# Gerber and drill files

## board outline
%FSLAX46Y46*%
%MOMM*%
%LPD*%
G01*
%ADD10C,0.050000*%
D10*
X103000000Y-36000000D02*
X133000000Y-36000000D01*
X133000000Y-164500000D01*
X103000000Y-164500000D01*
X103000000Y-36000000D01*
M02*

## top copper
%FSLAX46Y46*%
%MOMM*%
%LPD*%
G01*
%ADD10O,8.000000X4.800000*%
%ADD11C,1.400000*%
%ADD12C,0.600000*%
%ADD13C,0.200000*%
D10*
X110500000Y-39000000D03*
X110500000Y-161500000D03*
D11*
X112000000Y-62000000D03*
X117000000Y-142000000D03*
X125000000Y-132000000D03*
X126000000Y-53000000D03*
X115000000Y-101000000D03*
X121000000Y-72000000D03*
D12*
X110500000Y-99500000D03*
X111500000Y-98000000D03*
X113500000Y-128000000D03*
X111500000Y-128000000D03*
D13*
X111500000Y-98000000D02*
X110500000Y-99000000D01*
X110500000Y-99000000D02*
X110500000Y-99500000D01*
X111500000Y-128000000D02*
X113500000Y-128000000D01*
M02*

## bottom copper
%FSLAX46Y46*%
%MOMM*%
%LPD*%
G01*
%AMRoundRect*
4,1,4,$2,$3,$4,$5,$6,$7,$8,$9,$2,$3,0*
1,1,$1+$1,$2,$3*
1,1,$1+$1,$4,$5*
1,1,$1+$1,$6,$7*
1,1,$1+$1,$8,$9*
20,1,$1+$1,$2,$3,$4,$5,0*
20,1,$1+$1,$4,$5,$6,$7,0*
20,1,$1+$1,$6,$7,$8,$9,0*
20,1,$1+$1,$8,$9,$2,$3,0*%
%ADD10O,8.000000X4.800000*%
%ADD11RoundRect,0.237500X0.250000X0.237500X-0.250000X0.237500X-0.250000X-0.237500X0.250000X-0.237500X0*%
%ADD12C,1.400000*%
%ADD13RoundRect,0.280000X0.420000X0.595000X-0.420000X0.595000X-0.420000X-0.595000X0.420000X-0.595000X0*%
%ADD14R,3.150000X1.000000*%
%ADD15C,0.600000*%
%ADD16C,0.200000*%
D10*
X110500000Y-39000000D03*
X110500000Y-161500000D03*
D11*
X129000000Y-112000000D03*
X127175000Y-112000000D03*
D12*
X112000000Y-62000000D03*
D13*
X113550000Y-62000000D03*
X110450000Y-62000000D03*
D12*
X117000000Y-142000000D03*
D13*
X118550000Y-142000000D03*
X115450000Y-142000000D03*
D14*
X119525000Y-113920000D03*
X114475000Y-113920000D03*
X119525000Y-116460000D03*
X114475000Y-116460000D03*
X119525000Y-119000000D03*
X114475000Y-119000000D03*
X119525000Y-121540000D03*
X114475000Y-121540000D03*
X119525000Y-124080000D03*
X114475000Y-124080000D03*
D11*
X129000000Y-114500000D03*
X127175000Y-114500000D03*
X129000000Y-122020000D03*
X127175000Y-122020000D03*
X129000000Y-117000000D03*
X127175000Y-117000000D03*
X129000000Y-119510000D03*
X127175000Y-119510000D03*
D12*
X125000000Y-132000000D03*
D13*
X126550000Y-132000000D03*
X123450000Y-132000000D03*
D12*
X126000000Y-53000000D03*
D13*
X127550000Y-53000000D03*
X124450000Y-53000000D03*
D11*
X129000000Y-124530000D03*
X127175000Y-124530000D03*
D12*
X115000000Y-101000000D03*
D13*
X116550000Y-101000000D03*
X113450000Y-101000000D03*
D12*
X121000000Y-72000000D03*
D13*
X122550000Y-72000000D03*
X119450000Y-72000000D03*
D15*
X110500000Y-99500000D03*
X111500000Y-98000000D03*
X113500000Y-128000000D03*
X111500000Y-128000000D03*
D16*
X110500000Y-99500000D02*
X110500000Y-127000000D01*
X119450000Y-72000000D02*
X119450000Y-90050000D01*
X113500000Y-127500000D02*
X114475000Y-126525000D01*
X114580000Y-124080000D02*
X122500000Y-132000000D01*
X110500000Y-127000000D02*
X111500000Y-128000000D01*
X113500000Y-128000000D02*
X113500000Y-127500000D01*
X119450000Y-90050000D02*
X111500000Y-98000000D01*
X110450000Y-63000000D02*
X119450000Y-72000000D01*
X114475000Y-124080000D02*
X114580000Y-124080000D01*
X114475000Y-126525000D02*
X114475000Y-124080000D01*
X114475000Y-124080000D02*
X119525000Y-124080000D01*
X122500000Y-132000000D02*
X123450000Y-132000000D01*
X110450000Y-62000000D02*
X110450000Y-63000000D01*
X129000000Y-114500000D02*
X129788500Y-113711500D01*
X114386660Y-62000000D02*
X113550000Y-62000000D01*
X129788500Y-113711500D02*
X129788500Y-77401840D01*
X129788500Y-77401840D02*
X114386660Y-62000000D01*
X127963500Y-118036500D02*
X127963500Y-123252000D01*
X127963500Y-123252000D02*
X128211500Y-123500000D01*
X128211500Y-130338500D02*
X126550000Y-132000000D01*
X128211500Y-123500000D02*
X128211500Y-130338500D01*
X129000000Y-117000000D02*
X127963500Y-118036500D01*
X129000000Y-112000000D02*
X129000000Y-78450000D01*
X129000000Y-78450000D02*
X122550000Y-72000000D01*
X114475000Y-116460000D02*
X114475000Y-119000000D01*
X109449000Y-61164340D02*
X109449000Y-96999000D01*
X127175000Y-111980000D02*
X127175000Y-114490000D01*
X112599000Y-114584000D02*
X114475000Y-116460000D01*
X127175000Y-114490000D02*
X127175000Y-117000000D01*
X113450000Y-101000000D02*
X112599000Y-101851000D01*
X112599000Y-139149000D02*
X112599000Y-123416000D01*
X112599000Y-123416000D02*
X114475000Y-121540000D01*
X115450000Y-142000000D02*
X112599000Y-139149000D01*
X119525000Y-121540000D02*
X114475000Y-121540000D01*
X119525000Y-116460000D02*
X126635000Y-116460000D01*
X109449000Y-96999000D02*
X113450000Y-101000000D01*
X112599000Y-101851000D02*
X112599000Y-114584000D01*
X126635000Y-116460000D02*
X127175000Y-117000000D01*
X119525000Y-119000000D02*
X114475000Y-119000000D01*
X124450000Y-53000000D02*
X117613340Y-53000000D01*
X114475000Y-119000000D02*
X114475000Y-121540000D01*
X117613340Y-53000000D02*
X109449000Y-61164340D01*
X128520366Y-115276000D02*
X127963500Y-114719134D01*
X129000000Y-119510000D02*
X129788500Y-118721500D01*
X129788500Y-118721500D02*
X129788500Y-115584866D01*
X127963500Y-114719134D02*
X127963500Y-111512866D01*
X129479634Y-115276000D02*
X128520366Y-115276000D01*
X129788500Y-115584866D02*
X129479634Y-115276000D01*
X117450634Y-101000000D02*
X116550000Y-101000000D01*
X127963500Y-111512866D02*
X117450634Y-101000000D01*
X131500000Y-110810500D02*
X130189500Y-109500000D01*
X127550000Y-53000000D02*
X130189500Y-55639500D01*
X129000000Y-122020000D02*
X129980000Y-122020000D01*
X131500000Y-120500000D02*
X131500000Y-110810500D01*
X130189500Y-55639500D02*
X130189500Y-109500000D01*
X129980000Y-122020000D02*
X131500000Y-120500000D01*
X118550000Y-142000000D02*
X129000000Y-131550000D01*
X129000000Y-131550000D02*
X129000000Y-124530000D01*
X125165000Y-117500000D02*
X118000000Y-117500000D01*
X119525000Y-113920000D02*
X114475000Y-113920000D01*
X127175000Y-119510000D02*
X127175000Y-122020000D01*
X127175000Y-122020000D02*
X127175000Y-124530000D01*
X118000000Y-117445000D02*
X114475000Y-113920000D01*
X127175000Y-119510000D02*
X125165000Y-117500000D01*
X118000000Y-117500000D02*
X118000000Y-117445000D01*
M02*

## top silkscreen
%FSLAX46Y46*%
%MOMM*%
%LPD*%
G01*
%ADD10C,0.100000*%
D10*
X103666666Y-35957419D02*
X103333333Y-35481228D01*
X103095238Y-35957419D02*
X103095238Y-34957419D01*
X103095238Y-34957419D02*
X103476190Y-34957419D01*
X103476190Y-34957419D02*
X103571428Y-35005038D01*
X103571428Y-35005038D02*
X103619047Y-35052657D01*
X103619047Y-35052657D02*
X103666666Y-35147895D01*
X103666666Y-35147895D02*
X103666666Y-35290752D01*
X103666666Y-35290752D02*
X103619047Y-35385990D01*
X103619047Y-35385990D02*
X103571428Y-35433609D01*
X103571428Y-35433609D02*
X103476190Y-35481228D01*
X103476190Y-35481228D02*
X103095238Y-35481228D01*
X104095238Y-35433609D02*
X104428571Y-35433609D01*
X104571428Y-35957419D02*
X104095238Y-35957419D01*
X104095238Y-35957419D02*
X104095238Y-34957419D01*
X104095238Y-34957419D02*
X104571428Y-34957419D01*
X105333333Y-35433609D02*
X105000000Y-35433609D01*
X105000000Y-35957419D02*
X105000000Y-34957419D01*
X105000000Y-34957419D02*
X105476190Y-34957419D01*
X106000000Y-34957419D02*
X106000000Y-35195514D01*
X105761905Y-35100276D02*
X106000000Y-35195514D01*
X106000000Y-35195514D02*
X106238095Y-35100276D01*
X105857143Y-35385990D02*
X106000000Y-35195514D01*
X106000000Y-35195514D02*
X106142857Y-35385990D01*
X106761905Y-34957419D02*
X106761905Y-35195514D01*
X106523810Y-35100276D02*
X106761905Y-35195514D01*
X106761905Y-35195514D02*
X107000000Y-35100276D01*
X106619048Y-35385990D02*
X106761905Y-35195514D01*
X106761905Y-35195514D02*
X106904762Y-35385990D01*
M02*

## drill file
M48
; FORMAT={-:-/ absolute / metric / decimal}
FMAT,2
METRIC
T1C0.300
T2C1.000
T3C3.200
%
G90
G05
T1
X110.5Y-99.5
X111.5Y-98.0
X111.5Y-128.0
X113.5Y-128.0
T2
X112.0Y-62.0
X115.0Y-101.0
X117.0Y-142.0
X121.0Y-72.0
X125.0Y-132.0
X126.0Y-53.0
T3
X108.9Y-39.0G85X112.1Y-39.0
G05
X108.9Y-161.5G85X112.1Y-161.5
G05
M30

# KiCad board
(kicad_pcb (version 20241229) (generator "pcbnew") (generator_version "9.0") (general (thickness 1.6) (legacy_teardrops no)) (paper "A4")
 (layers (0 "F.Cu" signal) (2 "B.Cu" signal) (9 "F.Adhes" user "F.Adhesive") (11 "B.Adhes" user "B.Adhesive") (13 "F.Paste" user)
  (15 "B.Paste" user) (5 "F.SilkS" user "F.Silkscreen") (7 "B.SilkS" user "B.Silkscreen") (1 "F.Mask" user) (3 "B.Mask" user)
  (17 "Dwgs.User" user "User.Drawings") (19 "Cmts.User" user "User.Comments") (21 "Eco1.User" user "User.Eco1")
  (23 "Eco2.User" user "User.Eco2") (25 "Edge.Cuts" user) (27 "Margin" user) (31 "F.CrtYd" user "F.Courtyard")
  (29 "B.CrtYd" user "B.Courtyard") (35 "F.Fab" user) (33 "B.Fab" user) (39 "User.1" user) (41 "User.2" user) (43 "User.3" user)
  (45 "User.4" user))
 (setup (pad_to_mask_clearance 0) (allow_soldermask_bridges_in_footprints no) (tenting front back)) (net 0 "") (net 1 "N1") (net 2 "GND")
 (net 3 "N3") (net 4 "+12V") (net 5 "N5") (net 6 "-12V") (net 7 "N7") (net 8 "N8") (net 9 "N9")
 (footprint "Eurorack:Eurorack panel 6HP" (layer "F.Cu") (at 103 36)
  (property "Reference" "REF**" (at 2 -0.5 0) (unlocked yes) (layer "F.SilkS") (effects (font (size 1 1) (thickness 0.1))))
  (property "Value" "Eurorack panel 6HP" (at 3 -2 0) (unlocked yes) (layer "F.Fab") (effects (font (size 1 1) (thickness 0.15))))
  (fp_rect (start 0 0) (end 30 128.5) (stroke (width 0.05) (type solid)) (fill no) (layer "Edge.Cuts"))
  (pad "" thru_hole oval (at 7.5 3) (size 8 4.8) (drill oval 6.4 3.2) (layers "*.Cu" "*.Mask") (remove_unused_layers no))
  (pad "" thru_hole oval (at 7.5 125.5) (size 8 4.8) (drill oval 6.4 3.2) (layers "*.Cu" "*.Mask") (remove_unused_layers no)))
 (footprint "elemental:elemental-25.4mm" (layer "B.Cu") (at 117.837802 149.513938 180)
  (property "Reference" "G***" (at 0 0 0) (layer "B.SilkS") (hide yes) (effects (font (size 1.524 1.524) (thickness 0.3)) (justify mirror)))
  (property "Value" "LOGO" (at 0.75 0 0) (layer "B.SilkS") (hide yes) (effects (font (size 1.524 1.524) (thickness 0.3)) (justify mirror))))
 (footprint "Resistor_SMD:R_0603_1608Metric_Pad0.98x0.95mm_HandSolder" (layer "B.Cu") (at 128.0875 112 180)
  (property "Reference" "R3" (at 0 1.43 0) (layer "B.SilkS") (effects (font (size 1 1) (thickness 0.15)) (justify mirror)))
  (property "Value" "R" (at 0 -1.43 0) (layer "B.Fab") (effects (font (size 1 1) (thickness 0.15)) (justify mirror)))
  (pad "1" smd roundrect (at -0.9125 0 180) (size 0.975 0.95) (layers "B.Cu" "B.Mask" "B.Paste") (roundrect_rratio 0.25) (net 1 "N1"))
  (pad "2" smd roundrect (at 0.9125 0 180) (size 0.975 0.95) (layers "B.Cu" "B.Mask" "B.Paste") (roundrect_rratio 0.25) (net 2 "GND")))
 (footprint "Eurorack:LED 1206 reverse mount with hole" (layer "B.Cu") (at 112 62 180)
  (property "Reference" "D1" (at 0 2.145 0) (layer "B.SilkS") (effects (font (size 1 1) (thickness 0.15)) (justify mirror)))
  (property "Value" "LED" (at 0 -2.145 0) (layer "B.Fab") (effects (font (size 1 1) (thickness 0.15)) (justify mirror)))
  (pad "" thru_hole circle (at 0 0 180) (size 1.4 1.4) (drill 1) (layers "*.Cu" "*.Mask") (remove_unused_layers no))
  (pad "1" smd roundrect (at -1.55 0 180) (size 1.4 1.75) (layers "B.Cu" "B.Mask" "B.Paste") (roundrect_rratio 0.2) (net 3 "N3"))
  (pad "2" smd roundrect (at 1.55 0 180) (size 1.4 1.75) (layers "B.Cu" "B.Mask" "B.Paste") (roundrect_rratio 0.2) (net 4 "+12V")))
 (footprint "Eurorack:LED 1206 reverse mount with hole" (layer "B.Cu") (at 117 142 180)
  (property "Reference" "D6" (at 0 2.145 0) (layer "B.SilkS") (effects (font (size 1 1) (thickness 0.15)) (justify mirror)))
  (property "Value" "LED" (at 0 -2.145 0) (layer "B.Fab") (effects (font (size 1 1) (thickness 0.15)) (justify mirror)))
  (pad "" thru_hole circle (at 0 0 180) (size 1.4 1.4) (drill 1) (layers "*.Cu" "*.Mask") (remove_unused_layers no))
  (pad "1" smd roundrect (at -1.55 0 180) (size 1.4 1.75) (layers "B.Cu" "B.Mask" "B.Paste") (roundrect_rratio 0.2) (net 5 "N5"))
  (pad "2" smd roundrect (at 1.55 0 180) (size 1.4 1.75) (layers "B.Cu" "B.Mask" "B.Paste") (roundrect_rratio 0.2) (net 2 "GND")))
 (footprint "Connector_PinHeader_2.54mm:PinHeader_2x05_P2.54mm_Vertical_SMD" (layer "B.Cu") (at 117 119 180)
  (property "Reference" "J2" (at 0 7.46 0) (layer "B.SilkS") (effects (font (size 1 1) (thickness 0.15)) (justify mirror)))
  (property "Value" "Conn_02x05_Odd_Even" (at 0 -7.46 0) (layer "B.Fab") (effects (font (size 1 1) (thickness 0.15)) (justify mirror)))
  (pad "1" smd rect (at -2.525 5.08 180) (size 3.15 1) (layers "B.Cu" "B.Mask" "B.Paste") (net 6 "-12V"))
  (pad "2" smd rect (at 2.525 5.08 180) (size 3.15 1) (layers "B.Cu" "B.Mask" "B.Paste") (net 6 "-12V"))
  (pad "3" smd rect (at -2.525 2.54 180) (size 3.15 1) (layers "B.Cu" "B.Mask" "B.Paste") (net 2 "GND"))
  (pad "4" smd rect (at 2.525 2.54 180) (size 3.15 1) (layers "B.Cu" "B.Mask" "B.Paste") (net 2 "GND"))
  (pad "5" smd rect (at -2.525 0 180) (size 3.15 1) (layers "B.Cu" "B.Mask" "B.Paste") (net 2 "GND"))
  (pad "6" smd rect (at 2.525 0 180) (size 3.15 1) (layers "B.Cu" "B.Mask" "B.Paste") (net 2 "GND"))
  (pad "7" smd rect (at -2.525 -2.54 180) (size 3.15 1) (layers "B.Cu" "B.Mask" "B.Paste") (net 2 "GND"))
  (pad "8" smd rect (at 2.525 -2.54 180) (size 3.15 1) (layers "B.Cu" "B.Mask" "B.Paste") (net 2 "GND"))
  (pad "9" smd rect (at -2.525 -5.08 180) (size 3.15 1) (layers "B.Cu" "B.Mask" "B.Paste") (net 4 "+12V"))
  (pad "10" smd rect (at 2.525 -5.08 180) (size 3.15 1) (layers "B.Cu" "B.Mask" "B.Paste") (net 4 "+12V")))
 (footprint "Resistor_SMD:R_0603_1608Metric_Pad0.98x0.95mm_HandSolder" (layer "B.Cu") (at 128.0875 114.5 180)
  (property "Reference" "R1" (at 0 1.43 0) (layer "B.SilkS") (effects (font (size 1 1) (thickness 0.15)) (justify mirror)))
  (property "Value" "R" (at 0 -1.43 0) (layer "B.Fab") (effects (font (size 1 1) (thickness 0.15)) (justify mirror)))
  (pad "1" smd roundrect (at -0.9125 0 180) (size 0.975 0.95) (layers "B.Cu" "B.Mask" "B.Paste") (roundrect_rratio 0.25) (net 3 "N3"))
  (pad "2" smd roundrect (at 0.9125 0 180) (size 0.975 0.95) (layers "B.Cu" "B.Mask" "B.Paste") (roundrect_rratio 0.25) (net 2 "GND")))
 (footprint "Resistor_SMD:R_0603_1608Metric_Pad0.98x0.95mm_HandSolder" (layer "B.Cu") (at 128.0875 122.02 180)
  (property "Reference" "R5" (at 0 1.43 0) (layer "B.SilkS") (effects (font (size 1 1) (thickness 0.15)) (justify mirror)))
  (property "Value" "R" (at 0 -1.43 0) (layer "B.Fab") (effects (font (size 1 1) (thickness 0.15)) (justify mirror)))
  (pad "1" smd roundrect (at -0.9125 0 180) (size 0.975 0.95) (layers "B.Cu" "B.Mask" "B.Paste") (roundrect_rratio 0.25) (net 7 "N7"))
  (pad "2" smd roundrect (at 0.9125 0 180) (size 0.975 0.95) (layers "B.Cu" "B.Mask" "B.Paste") (roundrect_rratio 0.25) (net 6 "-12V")))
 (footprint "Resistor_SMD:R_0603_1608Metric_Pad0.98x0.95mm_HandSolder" (layer "B.Cu") (at 128.0875 117 180)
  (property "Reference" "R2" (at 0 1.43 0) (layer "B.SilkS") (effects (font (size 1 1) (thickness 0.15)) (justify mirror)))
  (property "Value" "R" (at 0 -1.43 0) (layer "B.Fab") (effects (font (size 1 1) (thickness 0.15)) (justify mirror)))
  (pad "1" smd roundrect (at -0.9125 0 180) (size 0.975 0.95) (layers "B.Cu" "B.Mask" "B.Paste") (roundrect_rratio 0.25) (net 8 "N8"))
  (pad "2" smd roundrect (at 0.9125 0 180) (size 0.975 0.95) (layers "B.Cu" "B.Mask" "B.Paste") (roundrect_rratio 0.25) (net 2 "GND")))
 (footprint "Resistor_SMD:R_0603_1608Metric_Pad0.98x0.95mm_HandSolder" (layer "B.Cu") (at 128.0875 119.51 180)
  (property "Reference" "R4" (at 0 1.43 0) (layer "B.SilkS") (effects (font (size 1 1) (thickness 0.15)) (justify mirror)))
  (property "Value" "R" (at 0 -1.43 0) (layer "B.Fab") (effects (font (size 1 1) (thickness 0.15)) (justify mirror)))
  (pad "1" smd roundrect (at -0.9125 0 180) (size 0.975 0.95) (layers "B.Cu" "B.Mask" "B.Paste") (roundrect_rratio 0.25) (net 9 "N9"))
  (pad "2" smd roundrect (at 0.9125 0 180) (size 0.975 0.95) (layers "B.Cu" "B.Mask" "B.Paste") (roundrect_rratio 0.25) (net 6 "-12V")))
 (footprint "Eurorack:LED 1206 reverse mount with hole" (layer "B.Cu") (at 125 132 180)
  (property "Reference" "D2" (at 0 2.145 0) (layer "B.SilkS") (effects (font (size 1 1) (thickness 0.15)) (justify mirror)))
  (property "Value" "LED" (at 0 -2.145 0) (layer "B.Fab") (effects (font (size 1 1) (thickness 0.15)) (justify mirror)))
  (pad "" thru_hole circle (at 0 0 180) (size 1.4 1.4) (drill 1) (layers "*.Cu" "*.Mask") (remove_unused_layers no))
  (pad "1" smd roundrect (at -1.55 0 180) (size 1.4 1.75) (layers "B.Cu" "B.Mask" "B.Paste") (roundrect_rratio 0.2) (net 8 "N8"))
  (pad "2" smd roundrect (at 1.55 0 180) (size 1.4 1.75) (layers "B.Cu" "B.Mask" "B.Paste") (roundrect_rratio 0.2) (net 4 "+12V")))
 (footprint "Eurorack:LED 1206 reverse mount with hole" (layer "B.Cu") (at 126 53 180)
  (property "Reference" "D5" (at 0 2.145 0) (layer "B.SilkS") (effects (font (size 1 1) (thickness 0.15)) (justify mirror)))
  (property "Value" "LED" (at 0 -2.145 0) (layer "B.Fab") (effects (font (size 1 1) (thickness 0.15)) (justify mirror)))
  (pad "" thru_hole circle (at 0 0 180) (size 1.4 1.4) (drill 1) (layers "*.Cu" "*.Mask") (remove_unused_layers no))
  (pad "1" smd roundrect (at -1.55 0 180) (size 1.4 1.75) (layers "B.Cu" "B.Mask" "B.Paste") (roundrect_rratio 0.2) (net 7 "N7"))
  (pad "2" smd roundrect (at 1.55 0 180) (size 1.4 1.75) (layers "B.Cu" "B.Mask" "B.Paste") (roundrect_rratio 0.2) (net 2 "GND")))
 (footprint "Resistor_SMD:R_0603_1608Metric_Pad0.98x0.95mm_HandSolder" (layer "B.Cu") (at 128.0875 124.53 180)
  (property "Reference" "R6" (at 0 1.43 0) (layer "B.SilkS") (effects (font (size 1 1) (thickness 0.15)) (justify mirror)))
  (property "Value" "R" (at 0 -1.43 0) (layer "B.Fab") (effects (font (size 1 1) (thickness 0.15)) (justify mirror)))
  (pad "1" smd roundrect (at -0.9125 0 180) (size 0.975 0.95) (layers "B.Cu" "B.Mask" "B.Paste") (roundrect_rratio 0.25) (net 5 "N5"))
  (pad "2" smd roundrect (at 0.9125 0 180) (size 0.975 0.95) (layers "B.Cu" "B.Mask" "B.Paste") (roundrect_rratio 0.25) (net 6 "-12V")))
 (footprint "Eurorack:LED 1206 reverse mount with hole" (layer "B.Cu") (at 115 101 180)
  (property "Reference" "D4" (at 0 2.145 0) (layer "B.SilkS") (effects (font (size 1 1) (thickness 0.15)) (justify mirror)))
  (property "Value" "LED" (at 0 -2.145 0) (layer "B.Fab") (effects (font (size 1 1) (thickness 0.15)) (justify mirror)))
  (pad "" thru_hole circle (at 0 0 180) (size 1.4 1.4) (drill 1) (layers "*.Cu" "*.Mask") (remove_unused_layers no))
  (pad "1" smd roundrect (at -1.55 0 180) (size 1.4 1.75) (layers "B.Cu" "B.Mask" "B.Paste") (roundrect_rratio 0.2) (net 9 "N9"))
  (pad "2" smd roundrect (at 1.55 0 180) (size 1.4 1.75) (layers "B.Cu" "B.Mask" "B.Paste") (roundrect_rratio 0.2) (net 2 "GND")))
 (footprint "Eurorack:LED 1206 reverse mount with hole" (layer "B.Cu") (at 121 72 180)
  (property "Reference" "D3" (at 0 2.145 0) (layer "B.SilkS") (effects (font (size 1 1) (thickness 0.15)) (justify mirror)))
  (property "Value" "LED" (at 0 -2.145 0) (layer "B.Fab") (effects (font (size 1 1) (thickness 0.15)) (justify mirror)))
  (pad "" thru_hole circle (at 0 0 180) (size 1.4 1.4) (drill 1) (layers "*.Cu" "*.Mask") (remove_unused_layers no))
  (pad "1" smd roundrect (at -1.55 0 180) (size 1.4 1.75) (layers "B.Cu" "B.Mask" "B.Paste") (roundrect_rratio 0.2) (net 1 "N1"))
  (pad "2" smd roundrect (at 1.55 0 180) (size 1.4 1.75) (layers "B.Cu" "B.Mask" "B.Paste") (roundrect_rratio 0.2) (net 4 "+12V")))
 (segment (start 111.5 98) (end 110.5 99) (width 0.2) (layer "F.Cu") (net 4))
 (segment (start 110.5 99) (end 110.5 99.5) (width 0.2) (layer "F.Cu") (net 4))
 (segment (start 111.5 128) (end 113.5 128) (width 0.2) (layer "F.Cu") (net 4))
 (via (at 110.5 99.5) (size 0.6) (drill 0.3) (layers "F.Cu" "B.Cu") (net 4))
 (via (at 111.5 98) (size 0.6) (drill 0.3) (layers "F.Cu" "B.Cu") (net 4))
 (via (at 113.5 128) (size 0.6) (drill 0.3) (layers "F.Cu" "B.Cu") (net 4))
 (via (at 111.5 128) (size 0.6) (drill 0.3) (layers "F.Cu" "B.Cu") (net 4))
 (segment (start 110.5 99.5) (end 110.5 127) (width 0.2) (layer "B.Cu") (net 4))
 (segment (start 119.45 72) (end 119.45 90.05) (width 0.2) (layer "B.Cu") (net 4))
 (segment (start 113.5 127.5) (end 114.475 126.525) (width 0.2) (layer "B.Cu") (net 4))
 (segment (start 114.58 124.08) (end 122.5 132) (width 0.2) (layer "B.Cu") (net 4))
 (segment (start 110.5 127) (end 111.5 128) (width 0.2) (layer "B.Cu") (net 4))
 (segment (start 113.5 128) (end 113.5 127.5) (width 0.2) (layer "B.Cu") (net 4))
 (segment (start 119.45 90.05) (end 111.5 98) (width 0.2) (layer "B.Cu") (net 4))
 (segment (start 110.45 63) (end 119.45 72) (width 0.2) (layer "B.Cu") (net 4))
 (segment (start 114.475 124.08) (end 114.58 124.08) (width 0.2) (layer "B.Cu") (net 4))
 (segment (start 114.475 126.525) (end 114.475 124.08) (width 0.2) (layer "B.Cu") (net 4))
 (segment (start 114.475 124.08) (end 119.525 124.08) (width 0.2) (layer "B.Cu") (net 4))
 (segment (start 122.5 132) (end 123.45 132) (width 0.2) (layer "B.Cu") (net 4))
 (segment (start 110.45 62) (end 110.45 63) (width 0.2) (layer "B.Cu") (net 4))
 (segment (start 129 114.5) (end 129.7885 113.7115) (width 0.2) (layer "B.Cu") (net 3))
 (segment (start 114.38666 62) (end 113.55 62) (width 0.2) (layer "B.Cu") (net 3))
 (segment (start 129.7885 113.7115) (end 129.7885 77.40184) (width 0.2) (layer "B.Cu") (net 3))
 (segment (start 129.7885 77.40184) (end 114.38666 62) (width 0.2) (layer "B.Cu") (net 3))
 (segment (start 127.9635 118.0365) (end 127.9635 123.252) (width 0.2) (layer "B.Cu") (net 8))
 (segment (start 127.9635 123.252) (end 128.2115 123.5) (width 0.2) (layer "B.Cu") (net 8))
 (segment (start 128.2115 130.3385) (end 126.55 132) (width 0.2) (layer "B.Cu") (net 8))
 (segment (start 128.2115 123.5) (end 128.2115 130.3385) (width 0.2) (layer "B.Cu") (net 8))
 (segment (start 129 117) (end 127.9635 118.0365) (width 0.2) (layer "B.Cu") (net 8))
 (segment (start 129 112) (end 129 78.45) (width 0.2) (layer "B.Cu") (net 1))
 (segment (start 129 78.45) (end 122.55 72) (width 0.2) (layer "B.Cu") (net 1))
 (segment (start 114.475 116.46) (end 114.475 119) (width 0.2) (layer "B.Cu") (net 2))
 (segment (start 109.449 61.16434) (end 109.449 96.999) (width 0.2) (layer "B.Cu") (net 2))
 (segment (start 127.175 111.98) (end 127.175 114.49) (width 0.2) (layer "B.Cu") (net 2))
 (segment (start 112.599 114.584) (end 114.475 116.46) (width 0.2) (layer "B.Cu") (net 2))
 (segment (start 127.175 114.49) (end 127.175 117) (width 0.2) (layer "B.Cu") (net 2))
 (segment (start 113.45 101) (end 112.599 101.851) (width 0.2) (layer "B.Cu") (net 2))
 (segment (start 112.599 139.149) (end 112.599 123.416) (width 0.2) (layer "B.Cu") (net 2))
 (segment (start 112.599 123.416) (end 114.475 121.54) (width 0.2) (layer "B.Cu") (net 2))
 (segment (start 115.45 142) (end 112.599 139.149) (width 0.2) (layer "B.Cu") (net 2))
 (segment (start 119.525 121.54) (end 114.475 121.54) (width 0.2) (layer "B.Cu") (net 2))
 (segment (start 119.525 116.46) (end 126.635 116.46) (width 0.2) (layer "B.Cu") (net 2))
 (segment (start 109.449 96.999) (end 113.45 101) (width 0.2) (layer "B.Cu") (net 2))
 (segment (start 112.599 101.851) (end 112.599 114.584) (width 0.2) (layer "B.Cu") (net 2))
 (segment (start 126.635 116.46) (end 127.175 117) (width 0.2) (layer "B.Cu") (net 2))
 (segment (start 119.525 119) (end 114.475 119) (width 0.2) (layer "B.Cu") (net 2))
 (segment (start 124.45 53) (end 117.61334 53) (width 0.2) (layer "B.Cu") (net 2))
 (segment (start 114.475 119) (end 114.475 121.54) (width 0.2) (layer "B.Cu") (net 2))
 (segment (start 117.61334 53) (end 109.449 61.16434) (width 0.2) (layer "B.Cu") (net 2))
 (segment (start 128.520366 115.276) (end 127.9635 114.719134) (width 0.2) (layer "B.Cu") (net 9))
 (segment (start 129 119.51) (end 129.7885 118.7215) (width 0.2) (layer "B.Cu") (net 9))
 (segment (start 129.7885 118.7215) (end 129.7885 115.584866) (width 0.2) (layer "B.Cu") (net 9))
 (segment (start 127.9635 114.719134) (end 127.9635 111.512866) (width 0.2) (layer "B.Cu") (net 9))
 (segment (start 129.479634 115.276) (end 128.520366 115.276) (width 0.2) (layer "B.Cu") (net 9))
 (segment (start 129.7885 115.584866) (end 129.479634 115.276) (width 0.2) (layer "B.Cu") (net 9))
 (segment (start 117.450634 101) (end 116.55 101) (width 0.2) (layer "B.Cu") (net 9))
 (segment (start 127.9635 111.512866) (end 117.450634 101) (width 0.2) (layer "B.Cu") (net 9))
 (segment (start 131.5 110.8105) (end 130.1895 109.5) (width 0.2) (layer "B.Cu") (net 7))
 (segment (start 127.55 53) (end 130.1895 55.6395) (width 0.2) (layer "B.Cu") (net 7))
 (segment (start 129 122.02) (end 129.98 122.02) (width 0.2) (layer "B.Cu") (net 7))
 (segment (start 131.5 120.5) (end 131.5 110.8105) (width 0.2) (layer "B.Cu") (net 7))
 (segment (start 130.1895 55.6395) (end 130.1895 109.5) (width 0.2) (layer "B.Cu") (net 7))
 (segment (start 129.98 122.02) (end 131.5 120.5) (width 0.2) (layer "B.Cu") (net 7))
 (segment (start 118.55 142) (end 129 131.55) (width 0.2) (layer "B.Cu") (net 5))
 (segment (start 129 131.55) (end 129 124.53) (width 0.2) (layer "B.Cu") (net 5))
 (segment (start 125.165 117.5) (end 118 117.5) (width 0.2) (layer "B.Cu") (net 6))
 (segment (start 119.525 113.92) (end 114.475 113.92) (width 0.2) (layer "B.Cu") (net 6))
 (segment (start 127.175 119.51) (end 127.175 122.02) (width 0.2) (layer "B.Cu") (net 6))
 (segment (start 127.175 122.02) (end 127.175 124.53) (width 0.2) (layer "B.Cu") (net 6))
 (segment (start 118 117.445) (end 114.475 113.92) (width 0.2) (layer "B.Cu") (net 6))
 (segment (start 127.175 119.51) (end 125.165 117.5) (width 0.2) (layer "B.Cu") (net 6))
 (segment (start 118 117.5) (end 118 117.445) (width 0.2) (layer "B.Cu") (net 6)))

